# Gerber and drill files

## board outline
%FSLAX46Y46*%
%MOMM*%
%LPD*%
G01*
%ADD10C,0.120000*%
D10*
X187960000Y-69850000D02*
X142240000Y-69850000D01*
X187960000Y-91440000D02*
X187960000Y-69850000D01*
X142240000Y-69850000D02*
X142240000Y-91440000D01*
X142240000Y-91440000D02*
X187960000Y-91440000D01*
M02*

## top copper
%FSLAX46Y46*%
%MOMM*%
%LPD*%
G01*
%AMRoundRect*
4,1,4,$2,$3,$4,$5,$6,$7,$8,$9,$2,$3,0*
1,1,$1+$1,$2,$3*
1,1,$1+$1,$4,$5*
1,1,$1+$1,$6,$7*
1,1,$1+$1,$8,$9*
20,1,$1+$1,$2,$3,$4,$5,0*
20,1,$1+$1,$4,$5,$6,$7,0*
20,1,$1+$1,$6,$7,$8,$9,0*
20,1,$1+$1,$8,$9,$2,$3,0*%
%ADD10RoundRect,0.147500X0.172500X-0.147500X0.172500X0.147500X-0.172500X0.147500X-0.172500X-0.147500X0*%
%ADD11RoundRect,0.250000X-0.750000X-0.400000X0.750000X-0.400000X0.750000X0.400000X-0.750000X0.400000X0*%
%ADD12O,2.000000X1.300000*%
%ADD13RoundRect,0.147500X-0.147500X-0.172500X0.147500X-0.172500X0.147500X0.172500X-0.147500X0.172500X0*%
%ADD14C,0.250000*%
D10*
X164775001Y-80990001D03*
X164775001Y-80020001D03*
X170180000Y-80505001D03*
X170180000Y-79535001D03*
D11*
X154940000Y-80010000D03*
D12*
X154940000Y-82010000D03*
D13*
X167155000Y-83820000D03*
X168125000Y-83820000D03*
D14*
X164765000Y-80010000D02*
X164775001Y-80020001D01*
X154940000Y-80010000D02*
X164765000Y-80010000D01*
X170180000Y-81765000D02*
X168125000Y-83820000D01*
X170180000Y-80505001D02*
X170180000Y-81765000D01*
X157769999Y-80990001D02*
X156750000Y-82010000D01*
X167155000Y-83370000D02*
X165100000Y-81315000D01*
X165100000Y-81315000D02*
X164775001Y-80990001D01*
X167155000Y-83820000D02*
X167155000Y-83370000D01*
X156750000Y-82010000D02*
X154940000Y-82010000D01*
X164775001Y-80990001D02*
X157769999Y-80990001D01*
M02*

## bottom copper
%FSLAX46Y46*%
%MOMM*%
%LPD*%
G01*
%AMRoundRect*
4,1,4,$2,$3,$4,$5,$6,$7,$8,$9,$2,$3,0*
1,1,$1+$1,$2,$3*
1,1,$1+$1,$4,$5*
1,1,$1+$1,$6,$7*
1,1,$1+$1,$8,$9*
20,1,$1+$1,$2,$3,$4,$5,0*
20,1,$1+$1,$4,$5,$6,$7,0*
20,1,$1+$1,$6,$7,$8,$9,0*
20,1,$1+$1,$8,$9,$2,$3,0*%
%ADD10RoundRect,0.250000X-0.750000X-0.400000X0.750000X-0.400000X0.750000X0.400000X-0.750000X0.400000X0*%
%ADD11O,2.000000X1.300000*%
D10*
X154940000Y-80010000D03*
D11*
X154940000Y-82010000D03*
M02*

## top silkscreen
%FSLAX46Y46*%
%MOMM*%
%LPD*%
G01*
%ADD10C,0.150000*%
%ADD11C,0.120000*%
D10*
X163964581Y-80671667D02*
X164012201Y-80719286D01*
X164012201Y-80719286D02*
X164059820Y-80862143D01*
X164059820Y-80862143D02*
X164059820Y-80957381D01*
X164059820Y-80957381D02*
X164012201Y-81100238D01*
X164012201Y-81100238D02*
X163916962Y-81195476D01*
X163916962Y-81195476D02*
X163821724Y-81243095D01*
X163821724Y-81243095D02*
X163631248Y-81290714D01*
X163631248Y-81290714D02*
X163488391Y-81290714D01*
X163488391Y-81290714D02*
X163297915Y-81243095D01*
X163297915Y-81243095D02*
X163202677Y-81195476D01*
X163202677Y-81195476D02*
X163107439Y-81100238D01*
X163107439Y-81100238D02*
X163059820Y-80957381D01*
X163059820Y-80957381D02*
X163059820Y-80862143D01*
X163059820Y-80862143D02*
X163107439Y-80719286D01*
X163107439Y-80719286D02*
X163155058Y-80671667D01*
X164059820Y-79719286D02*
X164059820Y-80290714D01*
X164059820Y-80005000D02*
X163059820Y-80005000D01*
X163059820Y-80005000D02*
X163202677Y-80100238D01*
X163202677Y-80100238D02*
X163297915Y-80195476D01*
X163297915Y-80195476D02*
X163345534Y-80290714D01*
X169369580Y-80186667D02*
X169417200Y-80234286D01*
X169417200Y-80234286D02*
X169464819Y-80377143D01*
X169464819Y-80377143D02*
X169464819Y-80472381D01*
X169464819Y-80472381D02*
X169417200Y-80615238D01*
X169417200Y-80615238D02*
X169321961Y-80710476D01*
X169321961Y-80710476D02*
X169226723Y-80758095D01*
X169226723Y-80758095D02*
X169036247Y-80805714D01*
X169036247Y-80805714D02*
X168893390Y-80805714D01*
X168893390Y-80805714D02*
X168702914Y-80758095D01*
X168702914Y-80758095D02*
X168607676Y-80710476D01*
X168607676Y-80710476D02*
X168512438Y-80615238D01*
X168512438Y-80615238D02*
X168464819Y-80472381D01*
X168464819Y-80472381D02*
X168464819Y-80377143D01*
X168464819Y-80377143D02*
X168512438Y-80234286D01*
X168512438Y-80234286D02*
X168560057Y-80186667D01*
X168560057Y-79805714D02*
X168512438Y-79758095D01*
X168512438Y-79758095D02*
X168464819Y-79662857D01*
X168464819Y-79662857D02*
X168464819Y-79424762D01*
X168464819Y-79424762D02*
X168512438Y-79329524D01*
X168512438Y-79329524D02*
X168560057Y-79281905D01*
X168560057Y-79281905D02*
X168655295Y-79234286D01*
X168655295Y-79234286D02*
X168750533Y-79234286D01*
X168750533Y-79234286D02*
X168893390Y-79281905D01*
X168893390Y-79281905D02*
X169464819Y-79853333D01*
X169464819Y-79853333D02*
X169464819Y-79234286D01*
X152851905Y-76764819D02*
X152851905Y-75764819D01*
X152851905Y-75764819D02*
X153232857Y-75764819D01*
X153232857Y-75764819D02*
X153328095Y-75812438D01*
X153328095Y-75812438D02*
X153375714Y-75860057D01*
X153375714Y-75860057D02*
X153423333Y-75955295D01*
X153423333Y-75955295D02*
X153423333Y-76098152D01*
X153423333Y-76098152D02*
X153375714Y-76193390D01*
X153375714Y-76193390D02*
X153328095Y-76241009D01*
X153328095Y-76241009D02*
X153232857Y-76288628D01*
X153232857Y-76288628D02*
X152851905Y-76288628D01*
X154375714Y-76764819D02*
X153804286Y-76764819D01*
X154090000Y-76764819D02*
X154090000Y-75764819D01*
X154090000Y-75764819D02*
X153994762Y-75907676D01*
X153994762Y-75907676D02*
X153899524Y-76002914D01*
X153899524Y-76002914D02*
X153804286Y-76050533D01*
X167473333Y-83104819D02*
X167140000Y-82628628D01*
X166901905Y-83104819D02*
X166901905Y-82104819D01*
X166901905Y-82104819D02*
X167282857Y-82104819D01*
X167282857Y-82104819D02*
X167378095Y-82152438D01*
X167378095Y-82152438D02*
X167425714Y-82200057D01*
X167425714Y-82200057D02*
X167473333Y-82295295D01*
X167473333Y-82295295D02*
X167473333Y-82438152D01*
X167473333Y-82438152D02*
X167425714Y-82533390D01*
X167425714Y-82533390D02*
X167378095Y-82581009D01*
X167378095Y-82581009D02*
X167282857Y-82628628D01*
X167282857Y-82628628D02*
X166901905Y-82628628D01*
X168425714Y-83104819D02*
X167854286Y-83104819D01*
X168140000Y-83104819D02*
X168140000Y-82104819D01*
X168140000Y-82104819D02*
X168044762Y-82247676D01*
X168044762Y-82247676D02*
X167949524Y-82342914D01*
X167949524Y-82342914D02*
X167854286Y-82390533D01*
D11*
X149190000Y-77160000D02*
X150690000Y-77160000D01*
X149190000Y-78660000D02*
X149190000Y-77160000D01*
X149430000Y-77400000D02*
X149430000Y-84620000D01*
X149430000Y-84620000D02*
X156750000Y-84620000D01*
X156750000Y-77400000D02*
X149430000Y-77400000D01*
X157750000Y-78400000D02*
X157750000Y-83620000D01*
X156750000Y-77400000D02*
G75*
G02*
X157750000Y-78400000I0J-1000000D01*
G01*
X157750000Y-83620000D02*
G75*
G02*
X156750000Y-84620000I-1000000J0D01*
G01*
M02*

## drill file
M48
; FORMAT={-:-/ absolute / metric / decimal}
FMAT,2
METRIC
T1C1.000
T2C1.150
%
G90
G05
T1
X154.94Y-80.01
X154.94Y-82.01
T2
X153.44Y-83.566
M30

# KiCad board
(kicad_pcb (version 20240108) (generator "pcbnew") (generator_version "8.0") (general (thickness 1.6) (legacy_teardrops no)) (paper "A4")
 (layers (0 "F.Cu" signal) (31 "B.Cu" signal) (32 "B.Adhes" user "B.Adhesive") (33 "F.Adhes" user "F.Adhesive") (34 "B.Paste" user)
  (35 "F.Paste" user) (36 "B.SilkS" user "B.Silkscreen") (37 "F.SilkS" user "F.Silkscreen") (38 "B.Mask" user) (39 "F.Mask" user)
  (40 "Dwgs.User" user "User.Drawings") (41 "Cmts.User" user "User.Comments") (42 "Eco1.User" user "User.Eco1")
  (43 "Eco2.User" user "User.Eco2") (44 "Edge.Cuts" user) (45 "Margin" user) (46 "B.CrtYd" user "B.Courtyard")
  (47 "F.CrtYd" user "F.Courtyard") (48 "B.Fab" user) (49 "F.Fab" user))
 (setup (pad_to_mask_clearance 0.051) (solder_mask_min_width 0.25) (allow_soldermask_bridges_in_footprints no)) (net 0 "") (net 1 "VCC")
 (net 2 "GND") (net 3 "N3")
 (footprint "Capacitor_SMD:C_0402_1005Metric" (layer "F.Cu") (at 164.775001 80.505001 90)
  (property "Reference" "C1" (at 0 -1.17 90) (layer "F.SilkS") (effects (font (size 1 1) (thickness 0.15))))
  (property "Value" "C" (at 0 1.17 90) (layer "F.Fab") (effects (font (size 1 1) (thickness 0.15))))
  (pad "1" smd roundrect (at -0.485 0 90) (size 0.59 0.64) (layers "F.Cu" "F.Paste" "F.Mask") (roundrect_rratio 0.25) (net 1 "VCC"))
  (pad "2" smd roundrect (at 0.485 0 90) (size 0.59 0.64) (layers "F.Cu" "F.Paste" "F.Mask") (roundrect_rratio 0.25) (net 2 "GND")))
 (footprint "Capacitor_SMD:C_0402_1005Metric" (layer "F.Cu") (at 170.18 80.020001 90)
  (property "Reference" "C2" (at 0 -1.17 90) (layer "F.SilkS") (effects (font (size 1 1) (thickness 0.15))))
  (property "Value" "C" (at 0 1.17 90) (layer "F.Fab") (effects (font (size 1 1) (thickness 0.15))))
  (pad "1" smd roundrect (at -0.485 0 90) (size 0.59 0.64) (layers "F.Cu" "F.Paste" "F.Mask") (roundrect_rratio 0.25) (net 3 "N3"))
  (pad "2" smd roundrect (at 0.485 0 90) (size 0.59 0.64) (layers "F.Cu" "F.Paste" "F.Mask") (roundrect_rratio 0.25) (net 2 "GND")))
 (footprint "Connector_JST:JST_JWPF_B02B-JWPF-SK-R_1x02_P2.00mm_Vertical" (layer "F.Cu") (at 154.94 80.01)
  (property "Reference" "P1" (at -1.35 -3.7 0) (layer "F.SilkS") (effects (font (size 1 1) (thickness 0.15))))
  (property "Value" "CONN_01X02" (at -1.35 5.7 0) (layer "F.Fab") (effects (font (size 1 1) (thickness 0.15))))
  (fp_line (start -5.75 -2.85) (end -4.25 -2.85) (stroke (width 0.12) (type solid)) (layer "F.SilkS"))
  (fp_line (start -5.75 -1.35) (end -5.75 -2.85) (stroke (width 0.12) (type solid)) (layer "F.SilkS"))
  (fp_line (start -5.51 -2.61) (end -5.51 4.61) (stroke (width 0.12) (type solid)) (layer "F.SilkS"))
  (fp_line (start -5.51 4.61) (end 1.81 4.61) (stroke (width 0.12) (type solid)) (layer "F.SilkS"))
  (fp_line (start 1.81 -2.61) (end -5.51 -2.61) (stroke (width 0.12) (type solid)) (layer "F.SilkS"))
  (fp_line (start 2.81 -1.61) (end 2.81 3.61) (stroke (width 0.12) (type solid)) (layer "F.SilkS"))
  (fp_arc (start 1.81 -2.61) (mid 2.517107 -2.317107) (end 2.81 -1.61) (stroke (width 0.12) (type solid)) (layer "F.SilkS"))
  (fp_arc (start 2.81 3.61) (mid 2.517107 4.317107) (end 1.81 4.61) (stroke (width 0.12) (type solid)) (layer "F.SilkS"))
  (pad "" np_thru_hole circle (at -1.5 3.556) (size 1.15 1.15) (drill 1.15) (layers "*.Cu" "*.Mask"))
  (pad "1" thru_hole roundrect (at 0 0) (size 2 1.3) (drill 1) (layers "*.Cu" "*.Mask") (remove_unused_layers no)
   (roundrect_rratio 0.192308) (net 2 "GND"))
  (pad "2" thru_hole oval (at 0 2) (size 2 1.3) (drill 1) (layers "*.Cu" "*.Mask") (remove_unused_layers no) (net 1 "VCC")))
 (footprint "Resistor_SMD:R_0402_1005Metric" (layer "F.Cu") (at 167.64 83.82)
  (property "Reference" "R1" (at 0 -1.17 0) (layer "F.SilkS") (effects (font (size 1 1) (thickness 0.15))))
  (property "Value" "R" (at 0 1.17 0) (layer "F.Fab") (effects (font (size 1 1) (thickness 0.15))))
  (pad "1" smd roundrect (at -0.485 0) (size 0.59 0.64) (layers "F.Cu" "F.Paste" "F.Mask") (roundrect_rratio 0.25) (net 1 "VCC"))
  (pad "2" smd roundrect (at 0.485 0) (size 0.59 0.64) (layers "F.Cu" "F.Paste" "F.Mask") (roundrect_rratio 0.25) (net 3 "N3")))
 (gr_line (start 187.96 69.85) (end 142.24 69.85) (stroke (width 0.12) (type solid)) (layer "Edge.Cuts"))
 (gr_line (start 187.96 91.44) (end 187.96 69.85) (stroke (width 0.12) (type solid)) (layer "Edge.Cuts"))
 (gr_line (start 142.24 69.85) (end 142.24 91.44) (stroke (width 0.12) (type solid)) (layer "Edge.Cuts"))
 (gr_line (start 142.24 91.44) (end 187.96 91.44) (stroke (width 0.12) (type solid)) (layer "Edge.Cuts"))
 (segment (start 164.765 80.01) (end 164.775001 80.020001) (width 0.25) (layer "F.Cu") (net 2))
 (segment (start 154.94 80.01) (end 164.765 80.01) (width 0.25) (layer "F.Cu") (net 2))
 (segment (start 170.18 81.765) (end 168.125 83.82) (width 0.25) (layer "F.Cu") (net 3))
 (segment (start 170.18 80.505001) (end 170.18 81.765) (width 0.25) (layer "F.Cu") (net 3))
 (segment (start 157.769999 80.990001) (end 156.75 82.01) (width 0.25) (layer "F.Cu") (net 1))
 (segment (start 167.155 83.37) (end 165.1 81.315) (width 0.25) (layer "F.Cu") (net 1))
 (segment (start 165.1 81.315) (end 164.775001 80.990001) (width 0.25) (layer "F.Cu") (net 1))
 (segment (start 167.155 83.82) (end 167.155 83.37) (width 0.25) (layer "F.Cu") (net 1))
 (segment (start 156.75 82.01) (end 154.94 82.01) (width 0.25) (layer "F.Cu") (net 1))
 (segment (start 164.775001 80.990001) (end 157.769999 80.990001) (width 0.25) (layer "F.Cu") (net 1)))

